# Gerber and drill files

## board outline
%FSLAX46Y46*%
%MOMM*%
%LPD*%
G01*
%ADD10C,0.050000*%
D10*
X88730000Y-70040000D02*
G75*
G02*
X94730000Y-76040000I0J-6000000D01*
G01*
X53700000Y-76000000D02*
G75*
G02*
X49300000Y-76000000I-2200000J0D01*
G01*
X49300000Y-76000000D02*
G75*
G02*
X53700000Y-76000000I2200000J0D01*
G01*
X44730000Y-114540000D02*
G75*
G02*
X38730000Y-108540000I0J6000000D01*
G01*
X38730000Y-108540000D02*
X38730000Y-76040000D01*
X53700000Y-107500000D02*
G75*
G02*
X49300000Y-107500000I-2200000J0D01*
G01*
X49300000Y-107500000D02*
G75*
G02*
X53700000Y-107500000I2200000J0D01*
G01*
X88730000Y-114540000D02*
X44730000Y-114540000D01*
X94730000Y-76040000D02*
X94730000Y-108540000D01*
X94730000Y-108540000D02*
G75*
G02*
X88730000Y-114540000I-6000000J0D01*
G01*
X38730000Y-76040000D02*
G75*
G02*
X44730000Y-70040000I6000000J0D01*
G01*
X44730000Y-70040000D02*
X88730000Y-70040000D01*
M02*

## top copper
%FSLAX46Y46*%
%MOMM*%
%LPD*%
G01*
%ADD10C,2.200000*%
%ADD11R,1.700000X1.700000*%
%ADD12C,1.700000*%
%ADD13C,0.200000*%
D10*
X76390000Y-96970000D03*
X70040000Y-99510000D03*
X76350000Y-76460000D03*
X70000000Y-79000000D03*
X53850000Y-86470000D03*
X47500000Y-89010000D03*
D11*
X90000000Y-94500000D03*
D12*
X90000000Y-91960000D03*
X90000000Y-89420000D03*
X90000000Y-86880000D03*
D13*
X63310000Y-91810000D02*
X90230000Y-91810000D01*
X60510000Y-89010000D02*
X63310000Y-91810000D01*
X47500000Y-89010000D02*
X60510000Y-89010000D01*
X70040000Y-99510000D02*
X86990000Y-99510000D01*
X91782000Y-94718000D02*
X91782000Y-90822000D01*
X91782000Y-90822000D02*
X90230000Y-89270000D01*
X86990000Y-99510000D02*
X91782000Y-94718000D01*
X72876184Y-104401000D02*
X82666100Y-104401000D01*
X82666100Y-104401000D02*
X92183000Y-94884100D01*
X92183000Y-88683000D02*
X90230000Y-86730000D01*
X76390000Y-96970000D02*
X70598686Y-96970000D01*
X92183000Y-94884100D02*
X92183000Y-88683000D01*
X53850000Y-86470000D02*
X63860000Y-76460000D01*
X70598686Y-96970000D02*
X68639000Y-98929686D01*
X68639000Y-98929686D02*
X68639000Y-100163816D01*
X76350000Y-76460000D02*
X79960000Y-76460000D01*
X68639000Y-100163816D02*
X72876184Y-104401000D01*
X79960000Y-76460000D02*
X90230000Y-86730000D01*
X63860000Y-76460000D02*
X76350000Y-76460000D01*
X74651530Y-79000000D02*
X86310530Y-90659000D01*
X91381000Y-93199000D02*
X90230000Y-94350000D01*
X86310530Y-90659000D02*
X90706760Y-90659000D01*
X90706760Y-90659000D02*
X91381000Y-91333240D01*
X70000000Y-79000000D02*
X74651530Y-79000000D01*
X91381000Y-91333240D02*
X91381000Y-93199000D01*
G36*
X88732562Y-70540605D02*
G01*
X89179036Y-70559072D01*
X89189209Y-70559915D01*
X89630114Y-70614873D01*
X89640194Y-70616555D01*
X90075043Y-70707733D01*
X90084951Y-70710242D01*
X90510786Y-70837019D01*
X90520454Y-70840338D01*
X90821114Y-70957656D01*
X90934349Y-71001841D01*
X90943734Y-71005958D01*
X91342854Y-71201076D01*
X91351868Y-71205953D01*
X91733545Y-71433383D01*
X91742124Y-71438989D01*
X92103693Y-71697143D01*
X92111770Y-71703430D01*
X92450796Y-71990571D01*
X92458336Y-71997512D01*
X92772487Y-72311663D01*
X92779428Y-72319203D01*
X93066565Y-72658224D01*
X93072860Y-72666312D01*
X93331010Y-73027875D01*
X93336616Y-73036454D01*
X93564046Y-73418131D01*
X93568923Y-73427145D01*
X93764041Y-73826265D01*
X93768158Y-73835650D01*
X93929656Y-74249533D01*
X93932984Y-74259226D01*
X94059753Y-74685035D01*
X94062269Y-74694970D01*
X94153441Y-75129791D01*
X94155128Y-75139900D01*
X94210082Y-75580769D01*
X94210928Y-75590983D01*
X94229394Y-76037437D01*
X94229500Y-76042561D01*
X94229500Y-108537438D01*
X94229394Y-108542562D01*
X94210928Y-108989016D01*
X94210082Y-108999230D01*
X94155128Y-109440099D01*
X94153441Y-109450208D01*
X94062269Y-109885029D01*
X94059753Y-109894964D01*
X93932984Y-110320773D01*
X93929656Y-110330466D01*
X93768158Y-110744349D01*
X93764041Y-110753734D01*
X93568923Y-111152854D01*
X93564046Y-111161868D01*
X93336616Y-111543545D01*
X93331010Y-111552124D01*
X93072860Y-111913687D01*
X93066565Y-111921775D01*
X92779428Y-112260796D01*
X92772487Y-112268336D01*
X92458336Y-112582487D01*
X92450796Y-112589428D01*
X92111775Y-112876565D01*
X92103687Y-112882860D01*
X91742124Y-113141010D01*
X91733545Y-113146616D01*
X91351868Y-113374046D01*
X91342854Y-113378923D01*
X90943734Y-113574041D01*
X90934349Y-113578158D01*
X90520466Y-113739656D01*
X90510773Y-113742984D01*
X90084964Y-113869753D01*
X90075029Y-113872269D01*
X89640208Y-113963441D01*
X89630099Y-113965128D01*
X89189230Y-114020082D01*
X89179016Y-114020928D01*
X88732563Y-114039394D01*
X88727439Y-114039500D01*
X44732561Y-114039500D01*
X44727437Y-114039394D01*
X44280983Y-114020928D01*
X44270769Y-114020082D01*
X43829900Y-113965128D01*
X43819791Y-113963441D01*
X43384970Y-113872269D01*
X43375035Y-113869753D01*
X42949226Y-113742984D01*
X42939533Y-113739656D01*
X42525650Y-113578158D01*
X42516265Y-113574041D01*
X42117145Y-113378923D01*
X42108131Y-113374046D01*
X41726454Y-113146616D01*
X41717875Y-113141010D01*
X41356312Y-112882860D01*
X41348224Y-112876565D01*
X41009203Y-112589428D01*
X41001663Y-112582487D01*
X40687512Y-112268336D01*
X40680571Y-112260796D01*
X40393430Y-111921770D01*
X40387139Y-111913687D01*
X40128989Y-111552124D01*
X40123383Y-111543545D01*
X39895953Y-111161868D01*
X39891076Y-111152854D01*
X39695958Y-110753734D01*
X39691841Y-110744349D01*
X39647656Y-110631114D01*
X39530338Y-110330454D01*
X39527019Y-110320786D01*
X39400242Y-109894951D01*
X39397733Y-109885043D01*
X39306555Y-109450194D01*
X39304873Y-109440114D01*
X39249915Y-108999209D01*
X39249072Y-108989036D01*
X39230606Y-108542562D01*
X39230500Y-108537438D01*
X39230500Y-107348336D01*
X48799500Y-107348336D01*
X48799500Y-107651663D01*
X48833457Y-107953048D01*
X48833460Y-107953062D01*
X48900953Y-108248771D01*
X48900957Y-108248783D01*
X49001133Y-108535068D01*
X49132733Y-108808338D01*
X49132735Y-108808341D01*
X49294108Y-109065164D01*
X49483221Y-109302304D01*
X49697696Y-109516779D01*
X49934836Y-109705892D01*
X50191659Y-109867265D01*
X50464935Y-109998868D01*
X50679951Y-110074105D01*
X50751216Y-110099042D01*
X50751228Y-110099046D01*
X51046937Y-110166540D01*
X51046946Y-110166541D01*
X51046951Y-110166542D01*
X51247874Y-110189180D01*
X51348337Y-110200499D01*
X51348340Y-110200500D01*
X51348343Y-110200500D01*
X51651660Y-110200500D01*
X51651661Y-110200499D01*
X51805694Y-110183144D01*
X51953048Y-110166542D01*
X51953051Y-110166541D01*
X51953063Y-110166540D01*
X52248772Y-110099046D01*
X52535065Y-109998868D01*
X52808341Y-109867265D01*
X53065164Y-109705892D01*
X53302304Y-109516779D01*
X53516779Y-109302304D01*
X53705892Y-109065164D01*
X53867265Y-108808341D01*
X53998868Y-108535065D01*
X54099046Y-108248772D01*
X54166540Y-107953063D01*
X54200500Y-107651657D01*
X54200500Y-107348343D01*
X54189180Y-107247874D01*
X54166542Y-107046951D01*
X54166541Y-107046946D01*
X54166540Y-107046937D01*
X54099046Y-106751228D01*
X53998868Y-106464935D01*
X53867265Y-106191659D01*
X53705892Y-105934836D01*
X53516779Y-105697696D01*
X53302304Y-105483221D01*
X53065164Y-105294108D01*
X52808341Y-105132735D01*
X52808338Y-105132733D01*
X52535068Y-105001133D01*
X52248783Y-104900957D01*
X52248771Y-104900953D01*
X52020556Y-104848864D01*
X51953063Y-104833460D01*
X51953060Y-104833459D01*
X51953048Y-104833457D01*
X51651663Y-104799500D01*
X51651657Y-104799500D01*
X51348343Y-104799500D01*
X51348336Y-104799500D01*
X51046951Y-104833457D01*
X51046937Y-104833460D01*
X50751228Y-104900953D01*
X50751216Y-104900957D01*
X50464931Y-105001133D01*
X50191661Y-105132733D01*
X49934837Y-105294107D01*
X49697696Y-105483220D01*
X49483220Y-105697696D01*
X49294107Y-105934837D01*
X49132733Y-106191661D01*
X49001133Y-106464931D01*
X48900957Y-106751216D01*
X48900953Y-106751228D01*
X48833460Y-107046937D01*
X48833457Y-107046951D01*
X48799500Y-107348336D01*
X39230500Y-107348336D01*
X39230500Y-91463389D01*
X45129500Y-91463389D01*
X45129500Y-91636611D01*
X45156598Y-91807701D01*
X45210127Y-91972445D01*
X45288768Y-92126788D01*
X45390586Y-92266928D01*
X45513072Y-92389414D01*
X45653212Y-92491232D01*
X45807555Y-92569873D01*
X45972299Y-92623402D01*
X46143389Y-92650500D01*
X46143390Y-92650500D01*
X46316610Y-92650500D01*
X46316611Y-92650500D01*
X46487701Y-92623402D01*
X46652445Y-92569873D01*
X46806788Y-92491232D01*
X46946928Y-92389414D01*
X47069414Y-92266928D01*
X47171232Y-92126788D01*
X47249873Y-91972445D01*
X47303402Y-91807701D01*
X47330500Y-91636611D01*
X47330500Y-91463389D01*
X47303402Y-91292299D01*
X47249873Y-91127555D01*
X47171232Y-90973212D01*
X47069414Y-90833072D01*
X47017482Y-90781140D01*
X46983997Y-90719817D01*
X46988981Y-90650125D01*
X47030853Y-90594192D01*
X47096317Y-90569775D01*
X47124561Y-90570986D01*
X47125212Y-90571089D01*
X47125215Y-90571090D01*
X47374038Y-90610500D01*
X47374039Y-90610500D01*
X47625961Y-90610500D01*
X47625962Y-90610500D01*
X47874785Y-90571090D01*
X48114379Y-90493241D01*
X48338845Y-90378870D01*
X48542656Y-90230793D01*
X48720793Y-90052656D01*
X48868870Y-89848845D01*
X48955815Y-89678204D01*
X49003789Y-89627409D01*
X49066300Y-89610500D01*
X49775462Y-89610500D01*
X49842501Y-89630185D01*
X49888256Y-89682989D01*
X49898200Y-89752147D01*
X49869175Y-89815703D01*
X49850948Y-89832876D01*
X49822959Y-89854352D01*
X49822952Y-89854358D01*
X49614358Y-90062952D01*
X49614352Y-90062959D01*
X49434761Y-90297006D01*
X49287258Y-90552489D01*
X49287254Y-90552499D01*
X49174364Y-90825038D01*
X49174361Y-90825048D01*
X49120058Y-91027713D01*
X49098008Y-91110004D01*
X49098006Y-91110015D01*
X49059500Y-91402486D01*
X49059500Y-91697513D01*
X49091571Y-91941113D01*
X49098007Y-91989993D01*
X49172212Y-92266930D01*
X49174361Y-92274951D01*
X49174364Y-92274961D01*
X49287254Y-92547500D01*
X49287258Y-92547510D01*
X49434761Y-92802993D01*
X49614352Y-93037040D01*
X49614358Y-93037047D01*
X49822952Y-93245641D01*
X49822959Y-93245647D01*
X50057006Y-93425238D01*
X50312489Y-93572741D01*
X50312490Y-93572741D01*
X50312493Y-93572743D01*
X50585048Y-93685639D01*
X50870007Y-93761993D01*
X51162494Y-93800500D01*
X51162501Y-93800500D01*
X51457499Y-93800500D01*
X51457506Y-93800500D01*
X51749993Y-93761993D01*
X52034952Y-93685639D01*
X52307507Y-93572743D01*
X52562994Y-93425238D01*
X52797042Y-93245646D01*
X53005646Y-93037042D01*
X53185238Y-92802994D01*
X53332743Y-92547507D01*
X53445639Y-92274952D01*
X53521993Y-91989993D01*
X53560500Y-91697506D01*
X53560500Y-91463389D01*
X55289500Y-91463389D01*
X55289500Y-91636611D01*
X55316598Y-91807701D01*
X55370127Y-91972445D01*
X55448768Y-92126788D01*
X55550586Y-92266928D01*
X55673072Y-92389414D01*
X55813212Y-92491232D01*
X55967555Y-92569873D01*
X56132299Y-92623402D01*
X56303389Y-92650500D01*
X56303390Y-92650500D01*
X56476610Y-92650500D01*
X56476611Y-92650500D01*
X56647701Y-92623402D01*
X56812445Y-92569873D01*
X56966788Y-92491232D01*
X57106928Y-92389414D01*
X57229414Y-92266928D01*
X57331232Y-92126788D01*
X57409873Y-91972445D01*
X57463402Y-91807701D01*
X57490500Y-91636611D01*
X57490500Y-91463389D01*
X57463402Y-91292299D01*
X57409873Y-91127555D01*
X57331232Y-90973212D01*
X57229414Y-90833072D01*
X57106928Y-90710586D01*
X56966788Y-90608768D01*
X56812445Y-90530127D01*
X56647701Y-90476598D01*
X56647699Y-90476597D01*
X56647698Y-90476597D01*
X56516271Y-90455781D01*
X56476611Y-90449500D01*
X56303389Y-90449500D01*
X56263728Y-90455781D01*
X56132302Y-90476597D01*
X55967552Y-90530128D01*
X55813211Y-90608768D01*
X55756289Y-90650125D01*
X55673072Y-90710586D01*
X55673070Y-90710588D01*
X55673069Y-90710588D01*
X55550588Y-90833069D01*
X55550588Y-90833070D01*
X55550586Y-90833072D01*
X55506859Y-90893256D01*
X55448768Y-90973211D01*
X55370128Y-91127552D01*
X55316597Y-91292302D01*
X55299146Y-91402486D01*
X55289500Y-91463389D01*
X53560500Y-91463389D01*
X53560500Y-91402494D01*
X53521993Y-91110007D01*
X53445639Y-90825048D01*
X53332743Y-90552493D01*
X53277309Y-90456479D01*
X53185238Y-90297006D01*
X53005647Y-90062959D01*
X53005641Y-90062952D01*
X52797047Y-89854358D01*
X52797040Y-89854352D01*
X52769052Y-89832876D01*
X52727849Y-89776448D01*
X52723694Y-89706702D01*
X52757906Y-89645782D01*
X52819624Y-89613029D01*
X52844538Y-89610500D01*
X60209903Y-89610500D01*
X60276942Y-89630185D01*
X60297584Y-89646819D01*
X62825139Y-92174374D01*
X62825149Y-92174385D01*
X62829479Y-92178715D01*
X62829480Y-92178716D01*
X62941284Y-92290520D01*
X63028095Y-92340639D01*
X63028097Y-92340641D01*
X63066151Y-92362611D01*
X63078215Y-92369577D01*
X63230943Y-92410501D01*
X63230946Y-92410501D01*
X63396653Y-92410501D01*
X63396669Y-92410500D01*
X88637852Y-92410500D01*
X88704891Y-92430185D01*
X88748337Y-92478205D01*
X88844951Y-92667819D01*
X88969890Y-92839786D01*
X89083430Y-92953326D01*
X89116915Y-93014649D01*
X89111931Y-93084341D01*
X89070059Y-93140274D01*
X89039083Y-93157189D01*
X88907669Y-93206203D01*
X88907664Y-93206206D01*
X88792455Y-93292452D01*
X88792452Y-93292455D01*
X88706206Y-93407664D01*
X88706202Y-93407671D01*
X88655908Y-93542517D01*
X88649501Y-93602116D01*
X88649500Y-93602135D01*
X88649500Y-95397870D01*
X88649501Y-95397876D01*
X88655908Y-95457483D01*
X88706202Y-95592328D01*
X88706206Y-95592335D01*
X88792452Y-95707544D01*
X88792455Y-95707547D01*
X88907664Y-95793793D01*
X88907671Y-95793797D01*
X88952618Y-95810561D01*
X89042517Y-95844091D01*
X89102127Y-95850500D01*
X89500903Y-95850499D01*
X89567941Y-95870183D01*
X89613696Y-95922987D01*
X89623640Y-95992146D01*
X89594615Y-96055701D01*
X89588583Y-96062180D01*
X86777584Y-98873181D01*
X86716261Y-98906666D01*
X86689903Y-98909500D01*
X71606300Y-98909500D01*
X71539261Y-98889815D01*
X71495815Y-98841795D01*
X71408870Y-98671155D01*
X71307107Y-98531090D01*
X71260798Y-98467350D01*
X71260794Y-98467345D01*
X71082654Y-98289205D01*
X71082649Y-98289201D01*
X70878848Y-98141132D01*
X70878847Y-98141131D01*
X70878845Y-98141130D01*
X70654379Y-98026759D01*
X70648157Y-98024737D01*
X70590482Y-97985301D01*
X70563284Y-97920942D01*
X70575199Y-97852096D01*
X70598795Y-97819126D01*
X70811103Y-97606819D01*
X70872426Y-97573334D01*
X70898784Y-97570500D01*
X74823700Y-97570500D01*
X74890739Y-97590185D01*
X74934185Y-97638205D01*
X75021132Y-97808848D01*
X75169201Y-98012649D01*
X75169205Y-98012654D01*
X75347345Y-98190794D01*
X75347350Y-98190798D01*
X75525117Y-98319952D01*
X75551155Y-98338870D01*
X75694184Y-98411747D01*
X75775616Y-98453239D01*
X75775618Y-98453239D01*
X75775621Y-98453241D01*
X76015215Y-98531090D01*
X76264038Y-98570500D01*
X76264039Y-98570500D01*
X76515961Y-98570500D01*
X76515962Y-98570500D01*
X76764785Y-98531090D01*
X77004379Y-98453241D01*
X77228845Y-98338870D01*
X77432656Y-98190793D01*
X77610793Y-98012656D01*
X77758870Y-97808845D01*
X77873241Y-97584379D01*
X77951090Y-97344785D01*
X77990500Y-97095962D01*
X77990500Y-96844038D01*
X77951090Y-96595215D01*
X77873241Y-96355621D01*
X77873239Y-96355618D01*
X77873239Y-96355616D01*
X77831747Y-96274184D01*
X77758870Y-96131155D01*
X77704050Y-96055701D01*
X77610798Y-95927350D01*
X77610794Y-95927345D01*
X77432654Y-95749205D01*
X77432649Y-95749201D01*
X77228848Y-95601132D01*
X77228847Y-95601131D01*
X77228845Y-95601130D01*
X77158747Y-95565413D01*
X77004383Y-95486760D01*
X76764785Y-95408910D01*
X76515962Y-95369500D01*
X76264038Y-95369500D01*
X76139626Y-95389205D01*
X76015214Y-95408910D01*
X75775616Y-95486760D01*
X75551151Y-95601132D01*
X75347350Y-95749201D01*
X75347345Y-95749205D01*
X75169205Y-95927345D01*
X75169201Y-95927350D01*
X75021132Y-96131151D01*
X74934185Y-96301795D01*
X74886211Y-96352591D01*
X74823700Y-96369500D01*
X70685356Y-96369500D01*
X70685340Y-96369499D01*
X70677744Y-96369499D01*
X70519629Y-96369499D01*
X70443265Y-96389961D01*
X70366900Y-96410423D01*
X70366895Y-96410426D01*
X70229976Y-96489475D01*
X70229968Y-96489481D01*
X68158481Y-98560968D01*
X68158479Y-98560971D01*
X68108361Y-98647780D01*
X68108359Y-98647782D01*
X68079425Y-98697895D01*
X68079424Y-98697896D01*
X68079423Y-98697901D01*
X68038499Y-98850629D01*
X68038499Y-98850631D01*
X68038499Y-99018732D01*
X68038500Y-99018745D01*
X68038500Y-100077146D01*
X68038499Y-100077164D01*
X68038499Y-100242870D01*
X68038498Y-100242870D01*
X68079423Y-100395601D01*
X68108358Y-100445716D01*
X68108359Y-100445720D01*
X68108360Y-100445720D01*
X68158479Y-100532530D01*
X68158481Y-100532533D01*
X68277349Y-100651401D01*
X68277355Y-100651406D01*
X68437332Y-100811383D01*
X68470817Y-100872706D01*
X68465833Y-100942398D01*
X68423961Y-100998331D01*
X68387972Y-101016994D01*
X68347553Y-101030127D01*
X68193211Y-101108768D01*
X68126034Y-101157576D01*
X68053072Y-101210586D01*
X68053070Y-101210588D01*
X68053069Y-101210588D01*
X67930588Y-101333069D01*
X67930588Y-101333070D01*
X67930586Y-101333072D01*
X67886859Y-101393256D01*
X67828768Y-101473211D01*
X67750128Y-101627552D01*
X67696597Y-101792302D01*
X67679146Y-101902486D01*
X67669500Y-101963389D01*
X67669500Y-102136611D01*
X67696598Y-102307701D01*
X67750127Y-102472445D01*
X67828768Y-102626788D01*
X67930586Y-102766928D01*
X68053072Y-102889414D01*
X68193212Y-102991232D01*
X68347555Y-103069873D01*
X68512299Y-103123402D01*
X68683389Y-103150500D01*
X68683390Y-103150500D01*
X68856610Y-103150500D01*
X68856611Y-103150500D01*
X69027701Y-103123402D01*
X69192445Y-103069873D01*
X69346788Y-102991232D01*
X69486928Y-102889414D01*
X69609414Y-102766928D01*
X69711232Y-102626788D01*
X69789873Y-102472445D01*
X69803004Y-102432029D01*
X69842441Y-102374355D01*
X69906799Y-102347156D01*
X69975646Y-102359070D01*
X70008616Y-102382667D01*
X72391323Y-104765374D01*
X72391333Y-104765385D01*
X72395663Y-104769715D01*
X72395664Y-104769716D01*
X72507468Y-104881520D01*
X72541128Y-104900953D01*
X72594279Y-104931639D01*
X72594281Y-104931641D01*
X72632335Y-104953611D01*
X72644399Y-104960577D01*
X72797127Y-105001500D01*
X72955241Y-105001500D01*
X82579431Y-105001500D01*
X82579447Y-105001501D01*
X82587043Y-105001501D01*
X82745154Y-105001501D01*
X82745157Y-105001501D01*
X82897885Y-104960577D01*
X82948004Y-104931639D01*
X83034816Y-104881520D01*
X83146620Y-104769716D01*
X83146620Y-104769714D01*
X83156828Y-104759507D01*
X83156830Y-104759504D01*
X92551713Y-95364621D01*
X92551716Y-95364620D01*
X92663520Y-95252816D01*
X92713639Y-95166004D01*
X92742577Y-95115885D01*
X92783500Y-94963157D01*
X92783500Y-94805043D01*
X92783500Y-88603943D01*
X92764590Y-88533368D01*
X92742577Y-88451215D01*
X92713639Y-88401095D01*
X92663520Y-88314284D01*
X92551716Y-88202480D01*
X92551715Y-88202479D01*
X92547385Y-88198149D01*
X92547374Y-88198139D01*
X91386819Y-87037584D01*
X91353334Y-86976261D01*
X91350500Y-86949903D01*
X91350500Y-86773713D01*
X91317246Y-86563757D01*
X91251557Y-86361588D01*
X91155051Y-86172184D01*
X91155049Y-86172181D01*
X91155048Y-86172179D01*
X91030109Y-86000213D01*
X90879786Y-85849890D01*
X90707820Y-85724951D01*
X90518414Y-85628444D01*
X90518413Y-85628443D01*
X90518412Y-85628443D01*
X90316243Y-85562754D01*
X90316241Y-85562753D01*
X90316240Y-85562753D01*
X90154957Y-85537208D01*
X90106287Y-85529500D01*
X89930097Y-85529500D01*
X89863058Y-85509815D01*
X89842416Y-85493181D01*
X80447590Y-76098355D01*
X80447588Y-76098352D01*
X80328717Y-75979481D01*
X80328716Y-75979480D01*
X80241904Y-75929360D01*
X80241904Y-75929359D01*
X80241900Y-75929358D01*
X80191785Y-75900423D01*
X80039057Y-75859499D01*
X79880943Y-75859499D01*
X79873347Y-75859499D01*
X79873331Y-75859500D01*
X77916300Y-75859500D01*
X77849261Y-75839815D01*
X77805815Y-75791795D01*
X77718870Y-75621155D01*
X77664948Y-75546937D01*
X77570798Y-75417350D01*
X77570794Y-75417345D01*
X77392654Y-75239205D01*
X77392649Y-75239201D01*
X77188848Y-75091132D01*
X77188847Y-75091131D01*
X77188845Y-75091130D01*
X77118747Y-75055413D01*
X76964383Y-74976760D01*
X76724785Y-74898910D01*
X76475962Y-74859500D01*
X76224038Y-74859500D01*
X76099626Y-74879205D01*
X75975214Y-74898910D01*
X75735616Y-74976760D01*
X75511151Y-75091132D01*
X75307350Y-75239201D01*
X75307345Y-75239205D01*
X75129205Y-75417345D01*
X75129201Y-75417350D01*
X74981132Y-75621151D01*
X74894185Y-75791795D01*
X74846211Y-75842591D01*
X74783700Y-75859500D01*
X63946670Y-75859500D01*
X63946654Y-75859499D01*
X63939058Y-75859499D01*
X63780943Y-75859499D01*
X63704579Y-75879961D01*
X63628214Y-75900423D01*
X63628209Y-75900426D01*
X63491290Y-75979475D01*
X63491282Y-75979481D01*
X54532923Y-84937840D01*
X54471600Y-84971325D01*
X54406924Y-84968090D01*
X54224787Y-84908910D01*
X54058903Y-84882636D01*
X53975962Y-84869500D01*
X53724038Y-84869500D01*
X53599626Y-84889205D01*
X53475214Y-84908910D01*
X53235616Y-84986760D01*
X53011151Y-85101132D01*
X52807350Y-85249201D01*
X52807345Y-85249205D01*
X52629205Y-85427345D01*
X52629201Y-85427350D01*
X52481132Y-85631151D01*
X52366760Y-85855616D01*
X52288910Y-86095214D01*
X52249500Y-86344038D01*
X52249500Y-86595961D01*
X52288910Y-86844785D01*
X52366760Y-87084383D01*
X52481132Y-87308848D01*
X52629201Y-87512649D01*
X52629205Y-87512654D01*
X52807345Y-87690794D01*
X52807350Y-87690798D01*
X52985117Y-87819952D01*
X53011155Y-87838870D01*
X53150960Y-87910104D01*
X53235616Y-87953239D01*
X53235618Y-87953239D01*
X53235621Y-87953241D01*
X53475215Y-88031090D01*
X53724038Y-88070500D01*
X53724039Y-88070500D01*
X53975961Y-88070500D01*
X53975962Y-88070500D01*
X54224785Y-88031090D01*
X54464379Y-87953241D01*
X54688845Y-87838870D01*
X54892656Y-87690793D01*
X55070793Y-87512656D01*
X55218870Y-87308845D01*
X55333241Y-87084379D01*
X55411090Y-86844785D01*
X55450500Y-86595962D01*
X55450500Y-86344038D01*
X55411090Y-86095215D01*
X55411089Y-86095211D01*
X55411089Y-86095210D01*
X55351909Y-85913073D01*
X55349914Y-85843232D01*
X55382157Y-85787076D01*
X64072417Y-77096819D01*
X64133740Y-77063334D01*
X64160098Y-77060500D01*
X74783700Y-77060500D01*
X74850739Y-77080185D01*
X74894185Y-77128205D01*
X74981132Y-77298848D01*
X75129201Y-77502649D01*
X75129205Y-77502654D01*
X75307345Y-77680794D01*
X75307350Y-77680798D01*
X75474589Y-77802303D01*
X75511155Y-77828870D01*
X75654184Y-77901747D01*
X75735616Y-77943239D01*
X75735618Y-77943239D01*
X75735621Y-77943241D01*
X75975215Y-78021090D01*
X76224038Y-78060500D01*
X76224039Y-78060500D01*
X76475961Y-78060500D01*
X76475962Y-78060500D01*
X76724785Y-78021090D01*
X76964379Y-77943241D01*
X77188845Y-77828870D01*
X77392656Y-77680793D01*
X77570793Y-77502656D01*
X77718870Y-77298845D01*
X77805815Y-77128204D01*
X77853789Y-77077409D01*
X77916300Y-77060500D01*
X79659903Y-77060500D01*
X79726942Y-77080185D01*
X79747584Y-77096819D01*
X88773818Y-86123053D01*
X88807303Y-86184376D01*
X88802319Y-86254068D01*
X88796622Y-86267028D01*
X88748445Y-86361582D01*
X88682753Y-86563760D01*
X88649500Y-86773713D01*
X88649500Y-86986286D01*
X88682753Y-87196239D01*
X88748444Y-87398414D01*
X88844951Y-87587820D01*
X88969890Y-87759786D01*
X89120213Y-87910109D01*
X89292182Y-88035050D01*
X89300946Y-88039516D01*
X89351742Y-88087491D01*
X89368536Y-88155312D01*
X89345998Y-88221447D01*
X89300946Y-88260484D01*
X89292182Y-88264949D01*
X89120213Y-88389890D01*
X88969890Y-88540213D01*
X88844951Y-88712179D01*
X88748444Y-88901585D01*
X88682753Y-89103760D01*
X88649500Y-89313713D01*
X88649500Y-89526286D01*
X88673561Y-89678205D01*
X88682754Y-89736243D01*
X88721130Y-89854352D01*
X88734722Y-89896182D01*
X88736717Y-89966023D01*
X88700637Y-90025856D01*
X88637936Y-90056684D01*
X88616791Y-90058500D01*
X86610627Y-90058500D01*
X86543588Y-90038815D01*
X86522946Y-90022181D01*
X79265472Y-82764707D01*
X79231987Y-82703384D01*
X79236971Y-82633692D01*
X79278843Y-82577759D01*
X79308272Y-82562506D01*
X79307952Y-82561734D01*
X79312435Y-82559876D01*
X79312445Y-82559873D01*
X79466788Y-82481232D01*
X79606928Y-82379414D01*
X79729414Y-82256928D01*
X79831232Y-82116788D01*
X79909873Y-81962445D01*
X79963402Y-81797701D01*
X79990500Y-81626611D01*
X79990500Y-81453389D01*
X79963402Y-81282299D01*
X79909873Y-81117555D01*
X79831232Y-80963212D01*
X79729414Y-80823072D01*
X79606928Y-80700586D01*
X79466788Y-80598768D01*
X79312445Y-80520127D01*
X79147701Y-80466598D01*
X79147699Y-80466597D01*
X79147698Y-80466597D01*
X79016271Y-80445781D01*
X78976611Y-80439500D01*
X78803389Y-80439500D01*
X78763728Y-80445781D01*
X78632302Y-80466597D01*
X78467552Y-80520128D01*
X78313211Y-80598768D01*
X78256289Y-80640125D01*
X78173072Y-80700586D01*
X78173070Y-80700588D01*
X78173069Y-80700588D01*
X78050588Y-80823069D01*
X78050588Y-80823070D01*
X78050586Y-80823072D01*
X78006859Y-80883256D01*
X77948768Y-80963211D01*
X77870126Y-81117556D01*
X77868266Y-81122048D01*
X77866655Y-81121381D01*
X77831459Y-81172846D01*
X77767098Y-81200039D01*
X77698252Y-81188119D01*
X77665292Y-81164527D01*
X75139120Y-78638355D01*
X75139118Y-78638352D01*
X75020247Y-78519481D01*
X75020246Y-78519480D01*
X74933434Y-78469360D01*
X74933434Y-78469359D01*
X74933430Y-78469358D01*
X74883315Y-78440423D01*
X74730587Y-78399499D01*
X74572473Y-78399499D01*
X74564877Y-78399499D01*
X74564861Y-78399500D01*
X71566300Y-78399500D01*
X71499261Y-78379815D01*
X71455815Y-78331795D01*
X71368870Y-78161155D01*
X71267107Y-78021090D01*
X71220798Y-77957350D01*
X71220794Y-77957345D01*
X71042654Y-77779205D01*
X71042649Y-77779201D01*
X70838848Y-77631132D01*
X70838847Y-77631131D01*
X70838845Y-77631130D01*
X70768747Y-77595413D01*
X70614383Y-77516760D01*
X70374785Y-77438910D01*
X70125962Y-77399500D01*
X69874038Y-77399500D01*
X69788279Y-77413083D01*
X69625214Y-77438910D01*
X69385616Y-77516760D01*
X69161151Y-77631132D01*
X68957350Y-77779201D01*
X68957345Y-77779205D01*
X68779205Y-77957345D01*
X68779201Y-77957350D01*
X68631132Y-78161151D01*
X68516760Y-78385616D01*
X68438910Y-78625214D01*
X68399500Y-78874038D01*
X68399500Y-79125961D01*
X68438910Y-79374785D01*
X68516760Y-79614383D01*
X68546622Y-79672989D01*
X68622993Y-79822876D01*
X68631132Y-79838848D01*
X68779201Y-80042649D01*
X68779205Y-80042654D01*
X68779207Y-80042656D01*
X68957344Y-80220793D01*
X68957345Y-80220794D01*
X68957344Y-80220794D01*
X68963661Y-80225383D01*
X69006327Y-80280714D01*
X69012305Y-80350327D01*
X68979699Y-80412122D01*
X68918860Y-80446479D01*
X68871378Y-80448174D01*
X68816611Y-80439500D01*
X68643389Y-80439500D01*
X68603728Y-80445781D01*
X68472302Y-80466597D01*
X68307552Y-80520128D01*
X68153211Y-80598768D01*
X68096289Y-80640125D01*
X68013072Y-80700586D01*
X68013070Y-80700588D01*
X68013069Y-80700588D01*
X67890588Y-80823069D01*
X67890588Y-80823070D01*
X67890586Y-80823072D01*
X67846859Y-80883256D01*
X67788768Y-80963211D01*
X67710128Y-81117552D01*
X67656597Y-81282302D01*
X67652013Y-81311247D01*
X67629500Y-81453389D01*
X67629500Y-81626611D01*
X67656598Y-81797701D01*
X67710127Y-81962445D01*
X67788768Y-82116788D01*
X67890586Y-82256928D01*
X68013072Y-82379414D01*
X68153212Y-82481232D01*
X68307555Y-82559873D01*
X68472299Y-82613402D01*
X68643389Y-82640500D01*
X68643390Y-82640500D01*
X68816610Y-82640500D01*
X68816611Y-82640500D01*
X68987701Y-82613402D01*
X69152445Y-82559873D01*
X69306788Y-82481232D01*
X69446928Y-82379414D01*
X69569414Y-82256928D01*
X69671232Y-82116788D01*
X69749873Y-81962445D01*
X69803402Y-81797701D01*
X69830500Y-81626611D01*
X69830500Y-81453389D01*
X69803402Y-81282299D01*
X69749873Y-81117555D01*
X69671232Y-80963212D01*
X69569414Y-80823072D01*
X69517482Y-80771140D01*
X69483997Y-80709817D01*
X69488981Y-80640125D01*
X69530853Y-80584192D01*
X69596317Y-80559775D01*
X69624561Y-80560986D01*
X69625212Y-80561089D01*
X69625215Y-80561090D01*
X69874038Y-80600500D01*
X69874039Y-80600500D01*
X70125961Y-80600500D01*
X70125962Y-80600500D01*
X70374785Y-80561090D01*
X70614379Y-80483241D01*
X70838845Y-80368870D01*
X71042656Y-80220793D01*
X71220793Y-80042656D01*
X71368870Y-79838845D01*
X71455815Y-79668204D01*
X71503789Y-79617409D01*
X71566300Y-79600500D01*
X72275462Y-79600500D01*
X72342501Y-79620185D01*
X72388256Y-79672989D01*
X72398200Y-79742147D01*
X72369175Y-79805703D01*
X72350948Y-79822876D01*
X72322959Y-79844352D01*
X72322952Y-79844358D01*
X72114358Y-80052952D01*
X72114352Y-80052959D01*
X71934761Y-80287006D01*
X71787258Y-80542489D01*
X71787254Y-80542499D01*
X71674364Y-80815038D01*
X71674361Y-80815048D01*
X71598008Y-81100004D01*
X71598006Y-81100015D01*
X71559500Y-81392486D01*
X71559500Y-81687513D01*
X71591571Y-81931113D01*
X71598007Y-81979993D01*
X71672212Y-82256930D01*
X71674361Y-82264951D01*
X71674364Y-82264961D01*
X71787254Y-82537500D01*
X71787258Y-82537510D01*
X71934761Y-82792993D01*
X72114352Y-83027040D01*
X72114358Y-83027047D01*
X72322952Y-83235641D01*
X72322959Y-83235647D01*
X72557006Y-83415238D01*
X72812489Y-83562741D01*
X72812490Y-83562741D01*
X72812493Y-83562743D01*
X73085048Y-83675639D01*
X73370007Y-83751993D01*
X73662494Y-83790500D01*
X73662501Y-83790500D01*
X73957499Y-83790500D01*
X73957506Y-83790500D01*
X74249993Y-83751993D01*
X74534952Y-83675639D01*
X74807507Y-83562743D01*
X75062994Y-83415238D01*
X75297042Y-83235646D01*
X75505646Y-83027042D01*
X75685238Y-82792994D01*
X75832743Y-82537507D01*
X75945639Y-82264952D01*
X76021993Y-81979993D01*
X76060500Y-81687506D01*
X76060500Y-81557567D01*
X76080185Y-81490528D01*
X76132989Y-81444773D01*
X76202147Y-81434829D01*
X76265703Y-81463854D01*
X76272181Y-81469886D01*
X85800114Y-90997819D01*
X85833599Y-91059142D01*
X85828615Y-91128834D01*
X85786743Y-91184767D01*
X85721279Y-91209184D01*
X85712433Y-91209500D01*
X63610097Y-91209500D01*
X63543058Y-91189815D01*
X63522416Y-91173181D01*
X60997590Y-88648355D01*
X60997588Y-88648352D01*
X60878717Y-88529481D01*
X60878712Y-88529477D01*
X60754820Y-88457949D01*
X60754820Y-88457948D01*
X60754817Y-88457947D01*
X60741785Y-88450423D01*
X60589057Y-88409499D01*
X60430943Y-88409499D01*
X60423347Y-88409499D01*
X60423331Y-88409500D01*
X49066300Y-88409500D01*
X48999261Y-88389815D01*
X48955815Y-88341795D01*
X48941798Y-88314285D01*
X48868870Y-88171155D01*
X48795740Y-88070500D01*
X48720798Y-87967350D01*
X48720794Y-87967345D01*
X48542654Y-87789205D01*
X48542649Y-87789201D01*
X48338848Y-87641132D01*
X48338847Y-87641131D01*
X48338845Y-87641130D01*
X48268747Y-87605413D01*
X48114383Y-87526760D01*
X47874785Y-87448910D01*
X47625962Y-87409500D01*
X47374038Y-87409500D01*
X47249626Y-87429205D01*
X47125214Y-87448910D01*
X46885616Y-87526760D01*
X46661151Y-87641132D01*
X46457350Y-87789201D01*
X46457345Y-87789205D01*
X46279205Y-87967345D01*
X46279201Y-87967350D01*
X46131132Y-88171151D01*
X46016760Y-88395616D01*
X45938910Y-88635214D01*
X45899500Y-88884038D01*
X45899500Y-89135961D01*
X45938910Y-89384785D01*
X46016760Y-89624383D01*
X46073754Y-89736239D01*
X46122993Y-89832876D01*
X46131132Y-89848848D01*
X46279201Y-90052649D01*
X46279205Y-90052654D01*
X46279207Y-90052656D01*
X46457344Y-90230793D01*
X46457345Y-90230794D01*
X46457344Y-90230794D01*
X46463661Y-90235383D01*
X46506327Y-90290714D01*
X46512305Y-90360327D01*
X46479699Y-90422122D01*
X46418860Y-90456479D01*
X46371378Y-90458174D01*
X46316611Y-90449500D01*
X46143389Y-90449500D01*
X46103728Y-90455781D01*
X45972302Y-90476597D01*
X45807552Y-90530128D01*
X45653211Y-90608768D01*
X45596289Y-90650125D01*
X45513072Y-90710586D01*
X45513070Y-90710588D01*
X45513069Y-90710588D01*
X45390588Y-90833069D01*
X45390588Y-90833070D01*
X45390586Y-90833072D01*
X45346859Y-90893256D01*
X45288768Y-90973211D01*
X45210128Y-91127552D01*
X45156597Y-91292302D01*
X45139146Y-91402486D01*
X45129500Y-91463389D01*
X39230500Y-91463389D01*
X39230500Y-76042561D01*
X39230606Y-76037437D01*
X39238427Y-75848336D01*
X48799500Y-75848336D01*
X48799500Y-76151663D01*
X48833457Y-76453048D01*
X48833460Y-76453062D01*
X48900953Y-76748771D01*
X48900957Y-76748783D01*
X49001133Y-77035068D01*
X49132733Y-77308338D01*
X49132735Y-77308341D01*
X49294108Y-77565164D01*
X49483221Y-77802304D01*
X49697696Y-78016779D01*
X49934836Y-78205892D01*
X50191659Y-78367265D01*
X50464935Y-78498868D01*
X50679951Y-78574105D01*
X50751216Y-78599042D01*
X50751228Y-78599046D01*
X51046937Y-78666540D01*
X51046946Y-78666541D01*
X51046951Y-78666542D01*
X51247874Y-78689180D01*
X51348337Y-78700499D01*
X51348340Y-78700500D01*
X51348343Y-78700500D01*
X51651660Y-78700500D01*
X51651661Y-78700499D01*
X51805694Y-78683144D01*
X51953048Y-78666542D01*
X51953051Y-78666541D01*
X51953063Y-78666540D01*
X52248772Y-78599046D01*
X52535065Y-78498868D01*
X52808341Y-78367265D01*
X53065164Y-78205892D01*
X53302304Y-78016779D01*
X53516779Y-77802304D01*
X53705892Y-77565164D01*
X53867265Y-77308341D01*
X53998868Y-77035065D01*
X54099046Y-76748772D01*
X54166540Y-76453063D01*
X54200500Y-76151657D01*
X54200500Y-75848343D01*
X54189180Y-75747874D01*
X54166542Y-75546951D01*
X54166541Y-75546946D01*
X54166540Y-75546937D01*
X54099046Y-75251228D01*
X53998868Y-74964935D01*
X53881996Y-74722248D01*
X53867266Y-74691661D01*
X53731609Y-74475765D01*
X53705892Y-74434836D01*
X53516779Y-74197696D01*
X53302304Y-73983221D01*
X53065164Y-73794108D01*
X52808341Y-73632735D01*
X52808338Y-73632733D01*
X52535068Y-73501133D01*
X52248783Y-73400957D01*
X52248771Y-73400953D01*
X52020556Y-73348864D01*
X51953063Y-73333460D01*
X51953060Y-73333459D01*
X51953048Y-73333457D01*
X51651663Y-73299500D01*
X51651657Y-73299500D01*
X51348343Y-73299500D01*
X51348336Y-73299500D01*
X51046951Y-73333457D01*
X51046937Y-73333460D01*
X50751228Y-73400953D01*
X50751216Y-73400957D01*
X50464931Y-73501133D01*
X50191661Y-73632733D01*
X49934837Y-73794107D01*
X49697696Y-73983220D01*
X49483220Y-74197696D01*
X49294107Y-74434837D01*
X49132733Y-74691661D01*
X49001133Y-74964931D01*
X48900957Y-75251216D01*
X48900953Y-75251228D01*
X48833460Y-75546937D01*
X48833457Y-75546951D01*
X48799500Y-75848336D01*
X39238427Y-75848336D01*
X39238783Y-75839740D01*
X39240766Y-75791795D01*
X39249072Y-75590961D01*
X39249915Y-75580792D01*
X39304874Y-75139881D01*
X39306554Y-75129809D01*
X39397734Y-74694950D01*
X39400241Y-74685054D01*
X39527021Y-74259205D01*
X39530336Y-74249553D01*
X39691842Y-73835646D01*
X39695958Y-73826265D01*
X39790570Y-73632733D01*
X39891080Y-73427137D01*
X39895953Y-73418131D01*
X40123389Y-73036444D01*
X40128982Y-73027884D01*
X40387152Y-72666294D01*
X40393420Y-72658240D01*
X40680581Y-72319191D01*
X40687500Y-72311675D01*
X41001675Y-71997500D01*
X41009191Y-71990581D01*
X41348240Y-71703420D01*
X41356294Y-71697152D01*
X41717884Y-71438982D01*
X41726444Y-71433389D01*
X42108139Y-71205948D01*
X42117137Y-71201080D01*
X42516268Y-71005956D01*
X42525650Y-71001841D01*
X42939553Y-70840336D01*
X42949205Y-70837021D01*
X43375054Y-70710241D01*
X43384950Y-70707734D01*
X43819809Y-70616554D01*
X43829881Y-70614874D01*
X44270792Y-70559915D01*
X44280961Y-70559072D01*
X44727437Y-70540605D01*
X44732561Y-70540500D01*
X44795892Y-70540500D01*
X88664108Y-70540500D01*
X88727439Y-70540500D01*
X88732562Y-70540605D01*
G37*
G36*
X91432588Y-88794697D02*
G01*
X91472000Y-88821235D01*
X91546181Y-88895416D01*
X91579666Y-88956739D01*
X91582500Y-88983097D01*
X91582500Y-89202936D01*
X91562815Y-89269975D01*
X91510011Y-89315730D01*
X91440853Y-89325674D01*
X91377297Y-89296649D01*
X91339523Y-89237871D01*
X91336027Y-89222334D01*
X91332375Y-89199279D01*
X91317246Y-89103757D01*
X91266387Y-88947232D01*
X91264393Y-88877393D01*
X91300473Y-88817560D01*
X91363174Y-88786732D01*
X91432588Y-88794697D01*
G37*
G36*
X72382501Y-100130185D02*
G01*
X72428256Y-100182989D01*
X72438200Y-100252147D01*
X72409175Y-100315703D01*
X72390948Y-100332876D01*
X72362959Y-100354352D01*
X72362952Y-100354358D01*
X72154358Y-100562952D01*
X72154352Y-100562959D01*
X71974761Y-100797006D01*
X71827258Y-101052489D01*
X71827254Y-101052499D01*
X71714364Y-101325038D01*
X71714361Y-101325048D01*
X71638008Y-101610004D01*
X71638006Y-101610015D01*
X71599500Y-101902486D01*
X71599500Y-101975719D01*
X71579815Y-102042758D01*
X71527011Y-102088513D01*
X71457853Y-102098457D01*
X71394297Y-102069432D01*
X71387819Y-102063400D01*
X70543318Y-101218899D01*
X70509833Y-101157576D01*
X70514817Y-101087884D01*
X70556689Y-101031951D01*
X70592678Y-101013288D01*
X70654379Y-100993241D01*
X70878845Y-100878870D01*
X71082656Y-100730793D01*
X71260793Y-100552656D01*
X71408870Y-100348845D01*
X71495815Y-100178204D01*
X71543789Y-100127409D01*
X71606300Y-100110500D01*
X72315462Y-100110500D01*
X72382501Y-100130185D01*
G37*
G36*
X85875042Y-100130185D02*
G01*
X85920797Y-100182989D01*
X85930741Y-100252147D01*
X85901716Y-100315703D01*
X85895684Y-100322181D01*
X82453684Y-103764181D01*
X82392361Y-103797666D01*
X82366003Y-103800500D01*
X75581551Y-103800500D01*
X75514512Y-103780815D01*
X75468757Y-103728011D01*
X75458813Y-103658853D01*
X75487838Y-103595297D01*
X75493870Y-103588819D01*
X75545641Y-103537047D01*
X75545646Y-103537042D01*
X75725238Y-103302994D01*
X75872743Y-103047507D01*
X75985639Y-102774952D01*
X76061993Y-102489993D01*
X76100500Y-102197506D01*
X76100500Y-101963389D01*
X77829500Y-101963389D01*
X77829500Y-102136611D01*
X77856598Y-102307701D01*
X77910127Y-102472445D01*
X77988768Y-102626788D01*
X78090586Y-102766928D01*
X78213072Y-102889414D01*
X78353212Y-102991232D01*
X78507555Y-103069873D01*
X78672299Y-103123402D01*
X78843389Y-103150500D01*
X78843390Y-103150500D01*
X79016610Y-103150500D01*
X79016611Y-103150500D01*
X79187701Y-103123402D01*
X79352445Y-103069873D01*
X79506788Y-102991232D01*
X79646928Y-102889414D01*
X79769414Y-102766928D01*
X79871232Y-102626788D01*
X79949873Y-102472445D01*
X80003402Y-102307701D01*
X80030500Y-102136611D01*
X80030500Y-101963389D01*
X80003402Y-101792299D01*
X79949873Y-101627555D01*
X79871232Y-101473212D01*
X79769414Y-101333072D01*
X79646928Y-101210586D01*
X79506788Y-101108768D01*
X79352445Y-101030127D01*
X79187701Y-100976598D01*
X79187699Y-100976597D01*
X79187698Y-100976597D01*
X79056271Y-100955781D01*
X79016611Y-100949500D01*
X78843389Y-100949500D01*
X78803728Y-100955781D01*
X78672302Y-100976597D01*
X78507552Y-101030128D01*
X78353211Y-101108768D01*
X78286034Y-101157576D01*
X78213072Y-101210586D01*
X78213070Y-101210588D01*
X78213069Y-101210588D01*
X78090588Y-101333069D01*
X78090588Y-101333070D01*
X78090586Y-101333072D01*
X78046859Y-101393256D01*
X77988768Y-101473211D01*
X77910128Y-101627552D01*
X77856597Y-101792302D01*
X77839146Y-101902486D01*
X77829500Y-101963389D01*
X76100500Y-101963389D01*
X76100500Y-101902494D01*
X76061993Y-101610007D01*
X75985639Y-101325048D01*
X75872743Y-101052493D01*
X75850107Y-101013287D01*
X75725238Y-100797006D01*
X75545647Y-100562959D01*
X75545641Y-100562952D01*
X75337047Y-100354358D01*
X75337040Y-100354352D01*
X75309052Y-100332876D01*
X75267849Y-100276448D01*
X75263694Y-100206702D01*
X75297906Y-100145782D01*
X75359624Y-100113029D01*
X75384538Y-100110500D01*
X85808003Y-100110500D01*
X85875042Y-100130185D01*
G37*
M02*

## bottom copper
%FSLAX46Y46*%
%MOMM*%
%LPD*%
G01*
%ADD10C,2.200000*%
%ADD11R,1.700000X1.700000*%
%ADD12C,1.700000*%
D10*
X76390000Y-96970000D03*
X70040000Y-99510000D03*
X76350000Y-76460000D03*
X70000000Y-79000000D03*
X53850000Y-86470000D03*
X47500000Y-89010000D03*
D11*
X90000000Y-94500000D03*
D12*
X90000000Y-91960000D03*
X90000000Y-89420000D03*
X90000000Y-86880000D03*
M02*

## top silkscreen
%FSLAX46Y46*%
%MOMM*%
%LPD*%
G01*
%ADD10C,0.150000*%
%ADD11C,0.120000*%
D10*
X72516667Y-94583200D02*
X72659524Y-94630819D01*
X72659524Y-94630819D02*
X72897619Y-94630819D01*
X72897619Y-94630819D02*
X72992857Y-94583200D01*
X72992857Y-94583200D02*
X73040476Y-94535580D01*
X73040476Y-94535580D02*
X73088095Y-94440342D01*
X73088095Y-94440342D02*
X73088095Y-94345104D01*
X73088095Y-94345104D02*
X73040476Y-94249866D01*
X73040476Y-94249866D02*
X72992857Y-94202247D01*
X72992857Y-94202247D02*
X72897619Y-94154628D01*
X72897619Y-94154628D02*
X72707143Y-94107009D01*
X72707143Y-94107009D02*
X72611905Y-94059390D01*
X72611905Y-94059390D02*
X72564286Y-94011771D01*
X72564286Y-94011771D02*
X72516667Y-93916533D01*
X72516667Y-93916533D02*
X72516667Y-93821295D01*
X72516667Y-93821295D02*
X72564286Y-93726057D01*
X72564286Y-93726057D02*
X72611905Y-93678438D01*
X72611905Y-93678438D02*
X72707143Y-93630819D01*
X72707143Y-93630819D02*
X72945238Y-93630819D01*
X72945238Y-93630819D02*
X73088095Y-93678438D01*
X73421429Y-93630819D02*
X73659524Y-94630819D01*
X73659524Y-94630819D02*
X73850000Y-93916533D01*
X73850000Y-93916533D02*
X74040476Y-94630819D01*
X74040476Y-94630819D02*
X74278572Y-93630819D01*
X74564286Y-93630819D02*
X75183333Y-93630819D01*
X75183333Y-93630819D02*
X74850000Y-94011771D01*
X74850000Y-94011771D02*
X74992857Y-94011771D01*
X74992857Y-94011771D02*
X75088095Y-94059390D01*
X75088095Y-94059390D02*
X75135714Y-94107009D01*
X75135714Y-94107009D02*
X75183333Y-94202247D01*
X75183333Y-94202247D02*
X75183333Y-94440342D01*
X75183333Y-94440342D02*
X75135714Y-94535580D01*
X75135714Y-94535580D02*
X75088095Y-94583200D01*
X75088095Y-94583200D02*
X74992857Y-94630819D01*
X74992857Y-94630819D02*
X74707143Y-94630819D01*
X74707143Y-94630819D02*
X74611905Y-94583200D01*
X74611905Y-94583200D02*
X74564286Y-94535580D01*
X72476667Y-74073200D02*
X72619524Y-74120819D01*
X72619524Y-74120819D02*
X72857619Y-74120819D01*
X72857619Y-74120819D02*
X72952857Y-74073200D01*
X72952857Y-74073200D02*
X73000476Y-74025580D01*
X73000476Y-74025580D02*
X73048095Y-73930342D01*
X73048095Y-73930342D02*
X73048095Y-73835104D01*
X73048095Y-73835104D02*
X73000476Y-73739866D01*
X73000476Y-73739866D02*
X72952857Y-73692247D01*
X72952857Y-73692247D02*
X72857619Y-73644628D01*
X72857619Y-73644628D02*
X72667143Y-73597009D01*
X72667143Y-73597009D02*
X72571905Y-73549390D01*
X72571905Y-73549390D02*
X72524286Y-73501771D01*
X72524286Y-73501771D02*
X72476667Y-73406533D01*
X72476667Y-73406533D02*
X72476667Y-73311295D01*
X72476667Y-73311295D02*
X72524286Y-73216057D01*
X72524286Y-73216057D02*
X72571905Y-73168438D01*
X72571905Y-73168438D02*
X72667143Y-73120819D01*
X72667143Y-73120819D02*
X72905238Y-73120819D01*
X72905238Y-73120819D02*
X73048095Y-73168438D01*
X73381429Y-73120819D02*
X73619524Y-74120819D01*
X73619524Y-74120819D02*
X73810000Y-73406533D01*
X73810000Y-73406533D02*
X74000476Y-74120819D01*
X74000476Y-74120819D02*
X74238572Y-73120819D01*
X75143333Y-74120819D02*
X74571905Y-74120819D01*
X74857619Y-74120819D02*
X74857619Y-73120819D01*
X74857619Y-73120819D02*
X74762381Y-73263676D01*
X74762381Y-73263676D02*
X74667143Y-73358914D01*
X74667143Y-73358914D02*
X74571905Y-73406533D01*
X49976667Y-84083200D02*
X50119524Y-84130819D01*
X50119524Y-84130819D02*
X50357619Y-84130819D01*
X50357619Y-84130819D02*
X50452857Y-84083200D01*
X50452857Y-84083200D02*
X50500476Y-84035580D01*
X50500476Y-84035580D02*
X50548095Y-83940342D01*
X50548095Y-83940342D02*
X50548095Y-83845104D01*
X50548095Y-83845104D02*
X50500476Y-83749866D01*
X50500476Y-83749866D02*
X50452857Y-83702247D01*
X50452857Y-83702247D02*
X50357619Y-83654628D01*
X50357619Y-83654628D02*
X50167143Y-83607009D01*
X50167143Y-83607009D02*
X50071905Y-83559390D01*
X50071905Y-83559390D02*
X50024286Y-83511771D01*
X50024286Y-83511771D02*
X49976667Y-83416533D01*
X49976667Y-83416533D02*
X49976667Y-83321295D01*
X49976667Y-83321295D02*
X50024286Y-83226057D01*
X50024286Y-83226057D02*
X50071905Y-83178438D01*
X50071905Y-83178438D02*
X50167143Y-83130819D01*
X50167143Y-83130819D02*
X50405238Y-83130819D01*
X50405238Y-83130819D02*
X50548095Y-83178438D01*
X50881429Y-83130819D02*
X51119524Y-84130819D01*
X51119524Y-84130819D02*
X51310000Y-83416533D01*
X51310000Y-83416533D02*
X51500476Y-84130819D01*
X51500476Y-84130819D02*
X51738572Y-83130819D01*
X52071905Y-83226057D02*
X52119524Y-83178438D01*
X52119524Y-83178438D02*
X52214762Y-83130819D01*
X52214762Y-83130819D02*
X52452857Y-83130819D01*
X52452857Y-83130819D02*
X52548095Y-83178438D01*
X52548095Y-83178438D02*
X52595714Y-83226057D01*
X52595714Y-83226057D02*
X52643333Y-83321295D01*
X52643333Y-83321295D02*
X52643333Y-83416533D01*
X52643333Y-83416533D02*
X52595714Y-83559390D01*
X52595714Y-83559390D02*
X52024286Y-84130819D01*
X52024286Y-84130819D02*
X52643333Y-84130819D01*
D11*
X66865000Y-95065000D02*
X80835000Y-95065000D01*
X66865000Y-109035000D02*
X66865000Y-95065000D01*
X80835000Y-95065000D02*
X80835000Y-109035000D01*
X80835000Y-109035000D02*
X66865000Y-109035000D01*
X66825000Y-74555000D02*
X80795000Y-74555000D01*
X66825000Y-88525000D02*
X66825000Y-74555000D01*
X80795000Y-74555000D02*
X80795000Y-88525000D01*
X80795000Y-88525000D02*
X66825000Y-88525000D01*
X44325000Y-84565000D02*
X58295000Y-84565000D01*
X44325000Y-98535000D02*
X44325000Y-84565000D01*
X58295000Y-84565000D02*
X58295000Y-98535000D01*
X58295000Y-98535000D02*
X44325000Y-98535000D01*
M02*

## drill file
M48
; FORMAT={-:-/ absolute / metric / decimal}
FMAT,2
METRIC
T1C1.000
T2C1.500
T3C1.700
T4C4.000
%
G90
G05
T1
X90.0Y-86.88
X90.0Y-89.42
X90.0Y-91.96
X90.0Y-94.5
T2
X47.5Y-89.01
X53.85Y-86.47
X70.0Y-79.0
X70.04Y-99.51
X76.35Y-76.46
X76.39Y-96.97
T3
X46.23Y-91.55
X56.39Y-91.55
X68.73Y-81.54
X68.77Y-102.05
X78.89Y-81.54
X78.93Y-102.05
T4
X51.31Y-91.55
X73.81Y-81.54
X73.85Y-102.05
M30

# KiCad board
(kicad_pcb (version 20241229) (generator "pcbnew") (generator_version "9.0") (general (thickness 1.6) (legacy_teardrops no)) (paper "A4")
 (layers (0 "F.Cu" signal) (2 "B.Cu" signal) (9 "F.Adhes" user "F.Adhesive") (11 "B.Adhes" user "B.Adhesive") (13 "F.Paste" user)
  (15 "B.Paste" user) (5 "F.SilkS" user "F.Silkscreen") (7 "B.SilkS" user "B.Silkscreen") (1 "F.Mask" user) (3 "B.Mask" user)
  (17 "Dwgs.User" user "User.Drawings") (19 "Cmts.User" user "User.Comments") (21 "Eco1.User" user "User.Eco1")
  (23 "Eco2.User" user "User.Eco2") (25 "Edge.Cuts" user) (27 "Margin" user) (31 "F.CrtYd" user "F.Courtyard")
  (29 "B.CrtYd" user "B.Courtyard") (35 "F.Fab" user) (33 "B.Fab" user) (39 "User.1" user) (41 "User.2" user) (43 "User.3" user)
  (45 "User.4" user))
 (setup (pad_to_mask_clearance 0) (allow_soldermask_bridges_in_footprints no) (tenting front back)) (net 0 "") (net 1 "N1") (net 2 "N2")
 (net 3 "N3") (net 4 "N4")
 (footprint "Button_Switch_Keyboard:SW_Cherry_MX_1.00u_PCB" (layer "F.Cu") (at 76.39 96.97)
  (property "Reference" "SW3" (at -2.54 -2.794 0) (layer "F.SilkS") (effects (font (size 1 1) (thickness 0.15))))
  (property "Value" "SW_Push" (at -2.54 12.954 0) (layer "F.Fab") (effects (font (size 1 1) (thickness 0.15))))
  (fp_line (start -9.525 -1.905) (end 4.445 -1.905) (stroke (width 0.12) (type solid)) (layer "F.SilkS"))
  (fp_line (start -9.525 12.065) (end -9.525 -1.905) (stroke (width 0.12) (type solid)) (layer "F.SilkS"))
  (fp_line (start 4.445 -1.905) (end 4.445 12.065) (stroke (width 0.12) (type solid)) (layer "F.SilkS"))
  (fp_line (start 4.445 12.065) (end -9.525 12.065) (stroke (width 0.12) (type solid)) (layer "F.SilkS"))
  (pad "" np_thru_hole circle (at -7.62 5.08) (size 1.7 1.7) (drill 1.7) (layers "*.Cu" "*.Mask"))
  (pad "" np_thru_hole circle (at -2.54 5.08) (size 4 4) (drill 4) (layers "*.Cu" "*.Mask"))
  (pad "" np_thru_hole circle (at 2.54 5.08) (size 1.7 1.7) (drill 1.7) (layers "*.Cu" "*.Mask"))
  (pad "1" thru_hole circle (at 0 0) (size 2.2 2.2) (drill 1.5) (layers "*.Cu" "*.Mask") (remove_unused_layers no) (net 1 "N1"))
  (pad "2" thru_hole circle (at -6.35 2.54) (size 2.2 2.2) (drill 1.5) (layers "*.Cu" "*.Mask") (remove_unused_layers no) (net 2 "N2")))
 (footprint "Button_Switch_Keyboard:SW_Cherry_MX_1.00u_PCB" (layer "F.Cu") (at 76.35 76.46)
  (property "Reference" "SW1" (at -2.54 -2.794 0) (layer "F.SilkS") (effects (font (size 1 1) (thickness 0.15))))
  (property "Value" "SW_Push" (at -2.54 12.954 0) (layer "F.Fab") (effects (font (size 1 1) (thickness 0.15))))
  (fp_line (start -9.525 -1.905) (end 4.445 -1.905) (stroke (width 0.12) (type solid)) (layer "F.SilkS"))
  (fp_line (start -9.525 12.065) (end -9.525 -1.905) (stroke (width 0.12) (type solid)) (layer "F.SilkS"))
  (fp_line (start 4.445 -1.905) (end 4.445 12.065) (stroke (width 0.12) (type solid)) (layer "F.SilkS"))
  (fp_line (start 4.445 12.065) (end -9.525 12.065) (stroke (width 0.12) (type solid)) (layer "F.SilkS"))
  (pad "" np_thru_hole circle (at -7.62 5.08) (size 1.7 1.7) (drill 1.7) (layers "*.Cu" "*.Mask"))
  (pad "" np_thru_hole circle (at -2.54 5.08) (size 4 4) (drill 4) (layers "*.Cu" "*.Mask"))
  (pad "" np_thru_hole circle (at 2.54 5.08) (size 1.7 1.7) (drill 1.7) (layers "*.Cu" "*.Mask"))
  (pad "1" thru_hole circle (at 0 0) (size 2.2 2.2) (drill 1.5) (layers "*.Cu" "*.Mask") (remove_unused_layers no) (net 1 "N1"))
  (pad "2" thru_hole circle (at -6.35 2.54) (size 2.2 2.2) (drill 1.5) (layers "*.Cu" "*.Mask") (remove_unused_layers no) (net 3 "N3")))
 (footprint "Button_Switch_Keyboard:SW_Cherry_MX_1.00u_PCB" (layer "F.Cu") (at 53.85 86.47)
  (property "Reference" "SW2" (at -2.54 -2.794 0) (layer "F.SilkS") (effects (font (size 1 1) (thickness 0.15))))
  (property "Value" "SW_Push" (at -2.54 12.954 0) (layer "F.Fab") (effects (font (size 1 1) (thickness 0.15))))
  (fp_line (start -9.525 -1.905) (end 4.445 -1.905) (stroke (width 0.12) (type solid)) (layer "F.SilkS"))
  (fp_line (start -9.525 12.065) (end -9.525 -1.905) (stroke (width 0.12) (type solid)) (layer "F.SilkS"))
  (fp_line (start 4.445 -1.905) (end 4.445 12.065) (stroke (width 0.12) (type solid)) (layer "F.SilkS"))
  (fp_line (start 4.445 12.065) (end -9.525 12.065) (stroke (width 0.12) (type solid)) (layer "F.SilkS"))
  (pad "" np_thru_hole circle (at -7.62 5.08) (size 1.7 1.7) (drill 1.7) (layers "*.Cu" "*.Mask"))
  (pad "" np_thru_hole circle (at -2.54 5.08) (size 4 4) (drill 4) (layers "*.Cu" "*.Mask"))
  (pad "" np_thru_hole circle (at 2.54 5.08) (size 1.7 1.7) (drill 1.7) (layers "*.Cu" "*.Mask"))
  (pad "1" thru_hole circle (at 0 0) (size 2.2 2.2) (drill 1.5) (layers "*.Cu" "*.Mask") (remove_unused_layers no) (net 1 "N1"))
  (pad "2" thru_hole circle (at -6.35 2.54) (size 2.2 2.2) (drill 1.5) (layers "*.Cu" "*.Mask") (remove_unused_layers no) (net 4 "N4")))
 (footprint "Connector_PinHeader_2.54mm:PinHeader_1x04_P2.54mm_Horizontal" (layer "B.Cu") (at 90 94.5)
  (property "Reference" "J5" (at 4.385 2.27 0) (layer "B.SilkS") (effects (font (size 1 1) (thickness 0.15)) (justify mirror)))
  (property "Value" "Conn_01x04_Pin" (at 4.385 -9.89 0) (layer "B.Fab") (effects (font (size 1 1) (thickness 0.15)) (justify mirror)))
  (pad "1" thru_hole rect (at 0 0) (size 1.7 1.7) (drill 1) (layers "*.Cu" "*.Mask") (remove_unused_layers no) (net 1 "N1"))
  (pad "2" thru_hole circle (at 0 -2.54) (size 1.7 1.7) (drill 1) (layers "*.Cu" "*.Mask") (remove_unused_layers no) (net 2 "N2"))
  (pad "3" thru_hole circle (at 0 -5.08) (size 1.7 1.7) (drill 1) (layers "*.Cu" "*.Mask") (remove_unused_layers no) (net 4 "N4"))
  (pad "4" thru_hole circle (at 0 -7.62) (size 1.7 1.7) (drill 1) (layers "*.Cu" "*.Mask") (remove_unused_layers no) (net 3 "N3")))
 (gr_arc (start 88.73 70.04) (mid 92.972641 71.797359) (end 94.73 76.04) (stroke (width 0.05) (type default)) (layer "Edge.Cuts"))
 (gr_circle (center 51.5 76) (end 53.7 76) (stroke (width 0.05) (type solid)) (fill no) (layer "Edge.Cuts"))
 (gr_arc (start 44.73 114.54) (mid 40.487359 112.782641) (end 38.73 108.54) (stroke (width 0.05) (type default)) (layer "Edge.Cuts"))
 (gr_line (start 38.73 108.54) (end 38.73 76.04) (stroke (width 0.05) (type default)) (layer "Edge.Cuts"))
 (gr_circle (center 51.5 107.5) (end 53.7 107.5) (stroke (width 0.05) (type solid)) (fill no) (layer "Edge.Cuts"))
 (gr_line (start 88.73 114.54) (end 44.73 114.54) (stroke (width 0.05) (type default)) (layer "Edge.Cuts"))
 (gr_line (start 94.73 76.04) (end 94.73 108.54) (stroke (width 0.05) (type default)) (layer "Edge.Cuts"))
 (gr_arc (start 94.73 108.54) (mid 92.972641 112.782641) (end 88.73 114.54) (stroke (width 0.05) (type default)) (layer "Edge.Cuts"))
 (gr_arc (start 38.73 76.04) (mid 40.487359 71.797359) (end 44.73 70.04) (stroke (width 0.05) (type default)) (layer "Edge.Cuts"))
 (gr_line (start 44.73 70.04) (end 88.73 70.04) (stroke (width 0.05) (type default)) (layer "Edge.Cuts"))
 (segment (start 63.31 91.81) (end 90.23 91.81) (width 0.2) (layer "F.Cu") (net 4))
 (segment (start 60.51 89.01) (end 63.31 91.81) (width 0.2) (layer "F.Cu") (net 4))
 (segment (start 47.5 89.01) (end 60.51 89.01) (width 0.2) (layer "F.Cu") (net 4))
 (segment (start 70.04 99.51) (end 86.99 99.51) (width 0.2) (layer "F.Cu") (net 2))
 (segment (start 91.782 94.718) (end 91.782 90.822) (width 0.2) (layer "F.Cu") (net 2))
 (segment (start 91.782 90.822) (end 90.23 89.27) (width 0.2) (layer "F.Cu") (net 2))
 (segment (start 86.99 99.51) (end 91.782 94.718) (width 0.2) (layer "F.Cu") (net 2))
 (segment (start 72.876184 104.401) (end 82.6661 104.401) (width 0.2) (layer "F.Cu") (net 1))
 (segment (start 82.6661 104.401) (end 92.183 94.8841) (width 0.2) (layer "F.Cu") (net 1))
 (segment (start 92.183 88.683) (end 90.23 86.73) (width 0.2) (layer "F.Cu") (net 1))
 (segment (start 76.39 96.97) (end 70.598686 96.97) (width 0.2) (layer "F.Cu") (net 1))
 (segment (start 92.183 94.8841) (end 92.183 88.683) (width 0.2) (layer "F.Cu") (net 1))
 (segment (start 53.85 86.47) (end 63.86 76.46) (width 0.2) (layer "F.Cu") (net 1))
 (segment (start 70.598686 96.97) (end 68.639 98.929686) (width 0.2) (layer "F.Cu") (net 1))
 (segment (start 68.639 98.929686) (end 68.639 100.163816) (width 0.2) (layer "F.Cu") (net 1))
 (segment (start 76.35 76.46) (end 79.96 76.46) (width 0.2) (layer "F.Cu") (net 1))
 (segment (start 68.639 100.163816) (end 72.876184 104.401) (width 0.2) (layer "F.Cu") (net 1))
 (segment (start 79.96 76.46) (end 90.23 86.73) (width 0.2) (layer "F.Cu") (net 1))
 (segment (start 63.86 76.46) (end 76.35 76.46) (width 0.2) (layer "F.Cu") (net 1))
 (segment (start 74.65153 79) (end 86.31053 90.659) (width 0.2) (layer "F.Cu") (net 3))
 (segment (start 91.381 93.199) (end 90.23 94.35) (width 0.2) (layer "F.Cu") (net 3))
 (segment (start 86.31053 90.659) (end 90.70676 90.659) (width 0.2) (layer "F.Cu") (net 3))
 (segment (start 90.70676 90.659) (end 91.381 91.33324) (width 0.2) (layer "F.Cu") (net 3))
 (segment (start 70 79) (end 74.65153 79) (width 0.2) (layer "F.Cu") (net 3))
 (segment (start 91.381 91.33324) (end 91.381 93.199) (width 0.2) (layer "F.Cu") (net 3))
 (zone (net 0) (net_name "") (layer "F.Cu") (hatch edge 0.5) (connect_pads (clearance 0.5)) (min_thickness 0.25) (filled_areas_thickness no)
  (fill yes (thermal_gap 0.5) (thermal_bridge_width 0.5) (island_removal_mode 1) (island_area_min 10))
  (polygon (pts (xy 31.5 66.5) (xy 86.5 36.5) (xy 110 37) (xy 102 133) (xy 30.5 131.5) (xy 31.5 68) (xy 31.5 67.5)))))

